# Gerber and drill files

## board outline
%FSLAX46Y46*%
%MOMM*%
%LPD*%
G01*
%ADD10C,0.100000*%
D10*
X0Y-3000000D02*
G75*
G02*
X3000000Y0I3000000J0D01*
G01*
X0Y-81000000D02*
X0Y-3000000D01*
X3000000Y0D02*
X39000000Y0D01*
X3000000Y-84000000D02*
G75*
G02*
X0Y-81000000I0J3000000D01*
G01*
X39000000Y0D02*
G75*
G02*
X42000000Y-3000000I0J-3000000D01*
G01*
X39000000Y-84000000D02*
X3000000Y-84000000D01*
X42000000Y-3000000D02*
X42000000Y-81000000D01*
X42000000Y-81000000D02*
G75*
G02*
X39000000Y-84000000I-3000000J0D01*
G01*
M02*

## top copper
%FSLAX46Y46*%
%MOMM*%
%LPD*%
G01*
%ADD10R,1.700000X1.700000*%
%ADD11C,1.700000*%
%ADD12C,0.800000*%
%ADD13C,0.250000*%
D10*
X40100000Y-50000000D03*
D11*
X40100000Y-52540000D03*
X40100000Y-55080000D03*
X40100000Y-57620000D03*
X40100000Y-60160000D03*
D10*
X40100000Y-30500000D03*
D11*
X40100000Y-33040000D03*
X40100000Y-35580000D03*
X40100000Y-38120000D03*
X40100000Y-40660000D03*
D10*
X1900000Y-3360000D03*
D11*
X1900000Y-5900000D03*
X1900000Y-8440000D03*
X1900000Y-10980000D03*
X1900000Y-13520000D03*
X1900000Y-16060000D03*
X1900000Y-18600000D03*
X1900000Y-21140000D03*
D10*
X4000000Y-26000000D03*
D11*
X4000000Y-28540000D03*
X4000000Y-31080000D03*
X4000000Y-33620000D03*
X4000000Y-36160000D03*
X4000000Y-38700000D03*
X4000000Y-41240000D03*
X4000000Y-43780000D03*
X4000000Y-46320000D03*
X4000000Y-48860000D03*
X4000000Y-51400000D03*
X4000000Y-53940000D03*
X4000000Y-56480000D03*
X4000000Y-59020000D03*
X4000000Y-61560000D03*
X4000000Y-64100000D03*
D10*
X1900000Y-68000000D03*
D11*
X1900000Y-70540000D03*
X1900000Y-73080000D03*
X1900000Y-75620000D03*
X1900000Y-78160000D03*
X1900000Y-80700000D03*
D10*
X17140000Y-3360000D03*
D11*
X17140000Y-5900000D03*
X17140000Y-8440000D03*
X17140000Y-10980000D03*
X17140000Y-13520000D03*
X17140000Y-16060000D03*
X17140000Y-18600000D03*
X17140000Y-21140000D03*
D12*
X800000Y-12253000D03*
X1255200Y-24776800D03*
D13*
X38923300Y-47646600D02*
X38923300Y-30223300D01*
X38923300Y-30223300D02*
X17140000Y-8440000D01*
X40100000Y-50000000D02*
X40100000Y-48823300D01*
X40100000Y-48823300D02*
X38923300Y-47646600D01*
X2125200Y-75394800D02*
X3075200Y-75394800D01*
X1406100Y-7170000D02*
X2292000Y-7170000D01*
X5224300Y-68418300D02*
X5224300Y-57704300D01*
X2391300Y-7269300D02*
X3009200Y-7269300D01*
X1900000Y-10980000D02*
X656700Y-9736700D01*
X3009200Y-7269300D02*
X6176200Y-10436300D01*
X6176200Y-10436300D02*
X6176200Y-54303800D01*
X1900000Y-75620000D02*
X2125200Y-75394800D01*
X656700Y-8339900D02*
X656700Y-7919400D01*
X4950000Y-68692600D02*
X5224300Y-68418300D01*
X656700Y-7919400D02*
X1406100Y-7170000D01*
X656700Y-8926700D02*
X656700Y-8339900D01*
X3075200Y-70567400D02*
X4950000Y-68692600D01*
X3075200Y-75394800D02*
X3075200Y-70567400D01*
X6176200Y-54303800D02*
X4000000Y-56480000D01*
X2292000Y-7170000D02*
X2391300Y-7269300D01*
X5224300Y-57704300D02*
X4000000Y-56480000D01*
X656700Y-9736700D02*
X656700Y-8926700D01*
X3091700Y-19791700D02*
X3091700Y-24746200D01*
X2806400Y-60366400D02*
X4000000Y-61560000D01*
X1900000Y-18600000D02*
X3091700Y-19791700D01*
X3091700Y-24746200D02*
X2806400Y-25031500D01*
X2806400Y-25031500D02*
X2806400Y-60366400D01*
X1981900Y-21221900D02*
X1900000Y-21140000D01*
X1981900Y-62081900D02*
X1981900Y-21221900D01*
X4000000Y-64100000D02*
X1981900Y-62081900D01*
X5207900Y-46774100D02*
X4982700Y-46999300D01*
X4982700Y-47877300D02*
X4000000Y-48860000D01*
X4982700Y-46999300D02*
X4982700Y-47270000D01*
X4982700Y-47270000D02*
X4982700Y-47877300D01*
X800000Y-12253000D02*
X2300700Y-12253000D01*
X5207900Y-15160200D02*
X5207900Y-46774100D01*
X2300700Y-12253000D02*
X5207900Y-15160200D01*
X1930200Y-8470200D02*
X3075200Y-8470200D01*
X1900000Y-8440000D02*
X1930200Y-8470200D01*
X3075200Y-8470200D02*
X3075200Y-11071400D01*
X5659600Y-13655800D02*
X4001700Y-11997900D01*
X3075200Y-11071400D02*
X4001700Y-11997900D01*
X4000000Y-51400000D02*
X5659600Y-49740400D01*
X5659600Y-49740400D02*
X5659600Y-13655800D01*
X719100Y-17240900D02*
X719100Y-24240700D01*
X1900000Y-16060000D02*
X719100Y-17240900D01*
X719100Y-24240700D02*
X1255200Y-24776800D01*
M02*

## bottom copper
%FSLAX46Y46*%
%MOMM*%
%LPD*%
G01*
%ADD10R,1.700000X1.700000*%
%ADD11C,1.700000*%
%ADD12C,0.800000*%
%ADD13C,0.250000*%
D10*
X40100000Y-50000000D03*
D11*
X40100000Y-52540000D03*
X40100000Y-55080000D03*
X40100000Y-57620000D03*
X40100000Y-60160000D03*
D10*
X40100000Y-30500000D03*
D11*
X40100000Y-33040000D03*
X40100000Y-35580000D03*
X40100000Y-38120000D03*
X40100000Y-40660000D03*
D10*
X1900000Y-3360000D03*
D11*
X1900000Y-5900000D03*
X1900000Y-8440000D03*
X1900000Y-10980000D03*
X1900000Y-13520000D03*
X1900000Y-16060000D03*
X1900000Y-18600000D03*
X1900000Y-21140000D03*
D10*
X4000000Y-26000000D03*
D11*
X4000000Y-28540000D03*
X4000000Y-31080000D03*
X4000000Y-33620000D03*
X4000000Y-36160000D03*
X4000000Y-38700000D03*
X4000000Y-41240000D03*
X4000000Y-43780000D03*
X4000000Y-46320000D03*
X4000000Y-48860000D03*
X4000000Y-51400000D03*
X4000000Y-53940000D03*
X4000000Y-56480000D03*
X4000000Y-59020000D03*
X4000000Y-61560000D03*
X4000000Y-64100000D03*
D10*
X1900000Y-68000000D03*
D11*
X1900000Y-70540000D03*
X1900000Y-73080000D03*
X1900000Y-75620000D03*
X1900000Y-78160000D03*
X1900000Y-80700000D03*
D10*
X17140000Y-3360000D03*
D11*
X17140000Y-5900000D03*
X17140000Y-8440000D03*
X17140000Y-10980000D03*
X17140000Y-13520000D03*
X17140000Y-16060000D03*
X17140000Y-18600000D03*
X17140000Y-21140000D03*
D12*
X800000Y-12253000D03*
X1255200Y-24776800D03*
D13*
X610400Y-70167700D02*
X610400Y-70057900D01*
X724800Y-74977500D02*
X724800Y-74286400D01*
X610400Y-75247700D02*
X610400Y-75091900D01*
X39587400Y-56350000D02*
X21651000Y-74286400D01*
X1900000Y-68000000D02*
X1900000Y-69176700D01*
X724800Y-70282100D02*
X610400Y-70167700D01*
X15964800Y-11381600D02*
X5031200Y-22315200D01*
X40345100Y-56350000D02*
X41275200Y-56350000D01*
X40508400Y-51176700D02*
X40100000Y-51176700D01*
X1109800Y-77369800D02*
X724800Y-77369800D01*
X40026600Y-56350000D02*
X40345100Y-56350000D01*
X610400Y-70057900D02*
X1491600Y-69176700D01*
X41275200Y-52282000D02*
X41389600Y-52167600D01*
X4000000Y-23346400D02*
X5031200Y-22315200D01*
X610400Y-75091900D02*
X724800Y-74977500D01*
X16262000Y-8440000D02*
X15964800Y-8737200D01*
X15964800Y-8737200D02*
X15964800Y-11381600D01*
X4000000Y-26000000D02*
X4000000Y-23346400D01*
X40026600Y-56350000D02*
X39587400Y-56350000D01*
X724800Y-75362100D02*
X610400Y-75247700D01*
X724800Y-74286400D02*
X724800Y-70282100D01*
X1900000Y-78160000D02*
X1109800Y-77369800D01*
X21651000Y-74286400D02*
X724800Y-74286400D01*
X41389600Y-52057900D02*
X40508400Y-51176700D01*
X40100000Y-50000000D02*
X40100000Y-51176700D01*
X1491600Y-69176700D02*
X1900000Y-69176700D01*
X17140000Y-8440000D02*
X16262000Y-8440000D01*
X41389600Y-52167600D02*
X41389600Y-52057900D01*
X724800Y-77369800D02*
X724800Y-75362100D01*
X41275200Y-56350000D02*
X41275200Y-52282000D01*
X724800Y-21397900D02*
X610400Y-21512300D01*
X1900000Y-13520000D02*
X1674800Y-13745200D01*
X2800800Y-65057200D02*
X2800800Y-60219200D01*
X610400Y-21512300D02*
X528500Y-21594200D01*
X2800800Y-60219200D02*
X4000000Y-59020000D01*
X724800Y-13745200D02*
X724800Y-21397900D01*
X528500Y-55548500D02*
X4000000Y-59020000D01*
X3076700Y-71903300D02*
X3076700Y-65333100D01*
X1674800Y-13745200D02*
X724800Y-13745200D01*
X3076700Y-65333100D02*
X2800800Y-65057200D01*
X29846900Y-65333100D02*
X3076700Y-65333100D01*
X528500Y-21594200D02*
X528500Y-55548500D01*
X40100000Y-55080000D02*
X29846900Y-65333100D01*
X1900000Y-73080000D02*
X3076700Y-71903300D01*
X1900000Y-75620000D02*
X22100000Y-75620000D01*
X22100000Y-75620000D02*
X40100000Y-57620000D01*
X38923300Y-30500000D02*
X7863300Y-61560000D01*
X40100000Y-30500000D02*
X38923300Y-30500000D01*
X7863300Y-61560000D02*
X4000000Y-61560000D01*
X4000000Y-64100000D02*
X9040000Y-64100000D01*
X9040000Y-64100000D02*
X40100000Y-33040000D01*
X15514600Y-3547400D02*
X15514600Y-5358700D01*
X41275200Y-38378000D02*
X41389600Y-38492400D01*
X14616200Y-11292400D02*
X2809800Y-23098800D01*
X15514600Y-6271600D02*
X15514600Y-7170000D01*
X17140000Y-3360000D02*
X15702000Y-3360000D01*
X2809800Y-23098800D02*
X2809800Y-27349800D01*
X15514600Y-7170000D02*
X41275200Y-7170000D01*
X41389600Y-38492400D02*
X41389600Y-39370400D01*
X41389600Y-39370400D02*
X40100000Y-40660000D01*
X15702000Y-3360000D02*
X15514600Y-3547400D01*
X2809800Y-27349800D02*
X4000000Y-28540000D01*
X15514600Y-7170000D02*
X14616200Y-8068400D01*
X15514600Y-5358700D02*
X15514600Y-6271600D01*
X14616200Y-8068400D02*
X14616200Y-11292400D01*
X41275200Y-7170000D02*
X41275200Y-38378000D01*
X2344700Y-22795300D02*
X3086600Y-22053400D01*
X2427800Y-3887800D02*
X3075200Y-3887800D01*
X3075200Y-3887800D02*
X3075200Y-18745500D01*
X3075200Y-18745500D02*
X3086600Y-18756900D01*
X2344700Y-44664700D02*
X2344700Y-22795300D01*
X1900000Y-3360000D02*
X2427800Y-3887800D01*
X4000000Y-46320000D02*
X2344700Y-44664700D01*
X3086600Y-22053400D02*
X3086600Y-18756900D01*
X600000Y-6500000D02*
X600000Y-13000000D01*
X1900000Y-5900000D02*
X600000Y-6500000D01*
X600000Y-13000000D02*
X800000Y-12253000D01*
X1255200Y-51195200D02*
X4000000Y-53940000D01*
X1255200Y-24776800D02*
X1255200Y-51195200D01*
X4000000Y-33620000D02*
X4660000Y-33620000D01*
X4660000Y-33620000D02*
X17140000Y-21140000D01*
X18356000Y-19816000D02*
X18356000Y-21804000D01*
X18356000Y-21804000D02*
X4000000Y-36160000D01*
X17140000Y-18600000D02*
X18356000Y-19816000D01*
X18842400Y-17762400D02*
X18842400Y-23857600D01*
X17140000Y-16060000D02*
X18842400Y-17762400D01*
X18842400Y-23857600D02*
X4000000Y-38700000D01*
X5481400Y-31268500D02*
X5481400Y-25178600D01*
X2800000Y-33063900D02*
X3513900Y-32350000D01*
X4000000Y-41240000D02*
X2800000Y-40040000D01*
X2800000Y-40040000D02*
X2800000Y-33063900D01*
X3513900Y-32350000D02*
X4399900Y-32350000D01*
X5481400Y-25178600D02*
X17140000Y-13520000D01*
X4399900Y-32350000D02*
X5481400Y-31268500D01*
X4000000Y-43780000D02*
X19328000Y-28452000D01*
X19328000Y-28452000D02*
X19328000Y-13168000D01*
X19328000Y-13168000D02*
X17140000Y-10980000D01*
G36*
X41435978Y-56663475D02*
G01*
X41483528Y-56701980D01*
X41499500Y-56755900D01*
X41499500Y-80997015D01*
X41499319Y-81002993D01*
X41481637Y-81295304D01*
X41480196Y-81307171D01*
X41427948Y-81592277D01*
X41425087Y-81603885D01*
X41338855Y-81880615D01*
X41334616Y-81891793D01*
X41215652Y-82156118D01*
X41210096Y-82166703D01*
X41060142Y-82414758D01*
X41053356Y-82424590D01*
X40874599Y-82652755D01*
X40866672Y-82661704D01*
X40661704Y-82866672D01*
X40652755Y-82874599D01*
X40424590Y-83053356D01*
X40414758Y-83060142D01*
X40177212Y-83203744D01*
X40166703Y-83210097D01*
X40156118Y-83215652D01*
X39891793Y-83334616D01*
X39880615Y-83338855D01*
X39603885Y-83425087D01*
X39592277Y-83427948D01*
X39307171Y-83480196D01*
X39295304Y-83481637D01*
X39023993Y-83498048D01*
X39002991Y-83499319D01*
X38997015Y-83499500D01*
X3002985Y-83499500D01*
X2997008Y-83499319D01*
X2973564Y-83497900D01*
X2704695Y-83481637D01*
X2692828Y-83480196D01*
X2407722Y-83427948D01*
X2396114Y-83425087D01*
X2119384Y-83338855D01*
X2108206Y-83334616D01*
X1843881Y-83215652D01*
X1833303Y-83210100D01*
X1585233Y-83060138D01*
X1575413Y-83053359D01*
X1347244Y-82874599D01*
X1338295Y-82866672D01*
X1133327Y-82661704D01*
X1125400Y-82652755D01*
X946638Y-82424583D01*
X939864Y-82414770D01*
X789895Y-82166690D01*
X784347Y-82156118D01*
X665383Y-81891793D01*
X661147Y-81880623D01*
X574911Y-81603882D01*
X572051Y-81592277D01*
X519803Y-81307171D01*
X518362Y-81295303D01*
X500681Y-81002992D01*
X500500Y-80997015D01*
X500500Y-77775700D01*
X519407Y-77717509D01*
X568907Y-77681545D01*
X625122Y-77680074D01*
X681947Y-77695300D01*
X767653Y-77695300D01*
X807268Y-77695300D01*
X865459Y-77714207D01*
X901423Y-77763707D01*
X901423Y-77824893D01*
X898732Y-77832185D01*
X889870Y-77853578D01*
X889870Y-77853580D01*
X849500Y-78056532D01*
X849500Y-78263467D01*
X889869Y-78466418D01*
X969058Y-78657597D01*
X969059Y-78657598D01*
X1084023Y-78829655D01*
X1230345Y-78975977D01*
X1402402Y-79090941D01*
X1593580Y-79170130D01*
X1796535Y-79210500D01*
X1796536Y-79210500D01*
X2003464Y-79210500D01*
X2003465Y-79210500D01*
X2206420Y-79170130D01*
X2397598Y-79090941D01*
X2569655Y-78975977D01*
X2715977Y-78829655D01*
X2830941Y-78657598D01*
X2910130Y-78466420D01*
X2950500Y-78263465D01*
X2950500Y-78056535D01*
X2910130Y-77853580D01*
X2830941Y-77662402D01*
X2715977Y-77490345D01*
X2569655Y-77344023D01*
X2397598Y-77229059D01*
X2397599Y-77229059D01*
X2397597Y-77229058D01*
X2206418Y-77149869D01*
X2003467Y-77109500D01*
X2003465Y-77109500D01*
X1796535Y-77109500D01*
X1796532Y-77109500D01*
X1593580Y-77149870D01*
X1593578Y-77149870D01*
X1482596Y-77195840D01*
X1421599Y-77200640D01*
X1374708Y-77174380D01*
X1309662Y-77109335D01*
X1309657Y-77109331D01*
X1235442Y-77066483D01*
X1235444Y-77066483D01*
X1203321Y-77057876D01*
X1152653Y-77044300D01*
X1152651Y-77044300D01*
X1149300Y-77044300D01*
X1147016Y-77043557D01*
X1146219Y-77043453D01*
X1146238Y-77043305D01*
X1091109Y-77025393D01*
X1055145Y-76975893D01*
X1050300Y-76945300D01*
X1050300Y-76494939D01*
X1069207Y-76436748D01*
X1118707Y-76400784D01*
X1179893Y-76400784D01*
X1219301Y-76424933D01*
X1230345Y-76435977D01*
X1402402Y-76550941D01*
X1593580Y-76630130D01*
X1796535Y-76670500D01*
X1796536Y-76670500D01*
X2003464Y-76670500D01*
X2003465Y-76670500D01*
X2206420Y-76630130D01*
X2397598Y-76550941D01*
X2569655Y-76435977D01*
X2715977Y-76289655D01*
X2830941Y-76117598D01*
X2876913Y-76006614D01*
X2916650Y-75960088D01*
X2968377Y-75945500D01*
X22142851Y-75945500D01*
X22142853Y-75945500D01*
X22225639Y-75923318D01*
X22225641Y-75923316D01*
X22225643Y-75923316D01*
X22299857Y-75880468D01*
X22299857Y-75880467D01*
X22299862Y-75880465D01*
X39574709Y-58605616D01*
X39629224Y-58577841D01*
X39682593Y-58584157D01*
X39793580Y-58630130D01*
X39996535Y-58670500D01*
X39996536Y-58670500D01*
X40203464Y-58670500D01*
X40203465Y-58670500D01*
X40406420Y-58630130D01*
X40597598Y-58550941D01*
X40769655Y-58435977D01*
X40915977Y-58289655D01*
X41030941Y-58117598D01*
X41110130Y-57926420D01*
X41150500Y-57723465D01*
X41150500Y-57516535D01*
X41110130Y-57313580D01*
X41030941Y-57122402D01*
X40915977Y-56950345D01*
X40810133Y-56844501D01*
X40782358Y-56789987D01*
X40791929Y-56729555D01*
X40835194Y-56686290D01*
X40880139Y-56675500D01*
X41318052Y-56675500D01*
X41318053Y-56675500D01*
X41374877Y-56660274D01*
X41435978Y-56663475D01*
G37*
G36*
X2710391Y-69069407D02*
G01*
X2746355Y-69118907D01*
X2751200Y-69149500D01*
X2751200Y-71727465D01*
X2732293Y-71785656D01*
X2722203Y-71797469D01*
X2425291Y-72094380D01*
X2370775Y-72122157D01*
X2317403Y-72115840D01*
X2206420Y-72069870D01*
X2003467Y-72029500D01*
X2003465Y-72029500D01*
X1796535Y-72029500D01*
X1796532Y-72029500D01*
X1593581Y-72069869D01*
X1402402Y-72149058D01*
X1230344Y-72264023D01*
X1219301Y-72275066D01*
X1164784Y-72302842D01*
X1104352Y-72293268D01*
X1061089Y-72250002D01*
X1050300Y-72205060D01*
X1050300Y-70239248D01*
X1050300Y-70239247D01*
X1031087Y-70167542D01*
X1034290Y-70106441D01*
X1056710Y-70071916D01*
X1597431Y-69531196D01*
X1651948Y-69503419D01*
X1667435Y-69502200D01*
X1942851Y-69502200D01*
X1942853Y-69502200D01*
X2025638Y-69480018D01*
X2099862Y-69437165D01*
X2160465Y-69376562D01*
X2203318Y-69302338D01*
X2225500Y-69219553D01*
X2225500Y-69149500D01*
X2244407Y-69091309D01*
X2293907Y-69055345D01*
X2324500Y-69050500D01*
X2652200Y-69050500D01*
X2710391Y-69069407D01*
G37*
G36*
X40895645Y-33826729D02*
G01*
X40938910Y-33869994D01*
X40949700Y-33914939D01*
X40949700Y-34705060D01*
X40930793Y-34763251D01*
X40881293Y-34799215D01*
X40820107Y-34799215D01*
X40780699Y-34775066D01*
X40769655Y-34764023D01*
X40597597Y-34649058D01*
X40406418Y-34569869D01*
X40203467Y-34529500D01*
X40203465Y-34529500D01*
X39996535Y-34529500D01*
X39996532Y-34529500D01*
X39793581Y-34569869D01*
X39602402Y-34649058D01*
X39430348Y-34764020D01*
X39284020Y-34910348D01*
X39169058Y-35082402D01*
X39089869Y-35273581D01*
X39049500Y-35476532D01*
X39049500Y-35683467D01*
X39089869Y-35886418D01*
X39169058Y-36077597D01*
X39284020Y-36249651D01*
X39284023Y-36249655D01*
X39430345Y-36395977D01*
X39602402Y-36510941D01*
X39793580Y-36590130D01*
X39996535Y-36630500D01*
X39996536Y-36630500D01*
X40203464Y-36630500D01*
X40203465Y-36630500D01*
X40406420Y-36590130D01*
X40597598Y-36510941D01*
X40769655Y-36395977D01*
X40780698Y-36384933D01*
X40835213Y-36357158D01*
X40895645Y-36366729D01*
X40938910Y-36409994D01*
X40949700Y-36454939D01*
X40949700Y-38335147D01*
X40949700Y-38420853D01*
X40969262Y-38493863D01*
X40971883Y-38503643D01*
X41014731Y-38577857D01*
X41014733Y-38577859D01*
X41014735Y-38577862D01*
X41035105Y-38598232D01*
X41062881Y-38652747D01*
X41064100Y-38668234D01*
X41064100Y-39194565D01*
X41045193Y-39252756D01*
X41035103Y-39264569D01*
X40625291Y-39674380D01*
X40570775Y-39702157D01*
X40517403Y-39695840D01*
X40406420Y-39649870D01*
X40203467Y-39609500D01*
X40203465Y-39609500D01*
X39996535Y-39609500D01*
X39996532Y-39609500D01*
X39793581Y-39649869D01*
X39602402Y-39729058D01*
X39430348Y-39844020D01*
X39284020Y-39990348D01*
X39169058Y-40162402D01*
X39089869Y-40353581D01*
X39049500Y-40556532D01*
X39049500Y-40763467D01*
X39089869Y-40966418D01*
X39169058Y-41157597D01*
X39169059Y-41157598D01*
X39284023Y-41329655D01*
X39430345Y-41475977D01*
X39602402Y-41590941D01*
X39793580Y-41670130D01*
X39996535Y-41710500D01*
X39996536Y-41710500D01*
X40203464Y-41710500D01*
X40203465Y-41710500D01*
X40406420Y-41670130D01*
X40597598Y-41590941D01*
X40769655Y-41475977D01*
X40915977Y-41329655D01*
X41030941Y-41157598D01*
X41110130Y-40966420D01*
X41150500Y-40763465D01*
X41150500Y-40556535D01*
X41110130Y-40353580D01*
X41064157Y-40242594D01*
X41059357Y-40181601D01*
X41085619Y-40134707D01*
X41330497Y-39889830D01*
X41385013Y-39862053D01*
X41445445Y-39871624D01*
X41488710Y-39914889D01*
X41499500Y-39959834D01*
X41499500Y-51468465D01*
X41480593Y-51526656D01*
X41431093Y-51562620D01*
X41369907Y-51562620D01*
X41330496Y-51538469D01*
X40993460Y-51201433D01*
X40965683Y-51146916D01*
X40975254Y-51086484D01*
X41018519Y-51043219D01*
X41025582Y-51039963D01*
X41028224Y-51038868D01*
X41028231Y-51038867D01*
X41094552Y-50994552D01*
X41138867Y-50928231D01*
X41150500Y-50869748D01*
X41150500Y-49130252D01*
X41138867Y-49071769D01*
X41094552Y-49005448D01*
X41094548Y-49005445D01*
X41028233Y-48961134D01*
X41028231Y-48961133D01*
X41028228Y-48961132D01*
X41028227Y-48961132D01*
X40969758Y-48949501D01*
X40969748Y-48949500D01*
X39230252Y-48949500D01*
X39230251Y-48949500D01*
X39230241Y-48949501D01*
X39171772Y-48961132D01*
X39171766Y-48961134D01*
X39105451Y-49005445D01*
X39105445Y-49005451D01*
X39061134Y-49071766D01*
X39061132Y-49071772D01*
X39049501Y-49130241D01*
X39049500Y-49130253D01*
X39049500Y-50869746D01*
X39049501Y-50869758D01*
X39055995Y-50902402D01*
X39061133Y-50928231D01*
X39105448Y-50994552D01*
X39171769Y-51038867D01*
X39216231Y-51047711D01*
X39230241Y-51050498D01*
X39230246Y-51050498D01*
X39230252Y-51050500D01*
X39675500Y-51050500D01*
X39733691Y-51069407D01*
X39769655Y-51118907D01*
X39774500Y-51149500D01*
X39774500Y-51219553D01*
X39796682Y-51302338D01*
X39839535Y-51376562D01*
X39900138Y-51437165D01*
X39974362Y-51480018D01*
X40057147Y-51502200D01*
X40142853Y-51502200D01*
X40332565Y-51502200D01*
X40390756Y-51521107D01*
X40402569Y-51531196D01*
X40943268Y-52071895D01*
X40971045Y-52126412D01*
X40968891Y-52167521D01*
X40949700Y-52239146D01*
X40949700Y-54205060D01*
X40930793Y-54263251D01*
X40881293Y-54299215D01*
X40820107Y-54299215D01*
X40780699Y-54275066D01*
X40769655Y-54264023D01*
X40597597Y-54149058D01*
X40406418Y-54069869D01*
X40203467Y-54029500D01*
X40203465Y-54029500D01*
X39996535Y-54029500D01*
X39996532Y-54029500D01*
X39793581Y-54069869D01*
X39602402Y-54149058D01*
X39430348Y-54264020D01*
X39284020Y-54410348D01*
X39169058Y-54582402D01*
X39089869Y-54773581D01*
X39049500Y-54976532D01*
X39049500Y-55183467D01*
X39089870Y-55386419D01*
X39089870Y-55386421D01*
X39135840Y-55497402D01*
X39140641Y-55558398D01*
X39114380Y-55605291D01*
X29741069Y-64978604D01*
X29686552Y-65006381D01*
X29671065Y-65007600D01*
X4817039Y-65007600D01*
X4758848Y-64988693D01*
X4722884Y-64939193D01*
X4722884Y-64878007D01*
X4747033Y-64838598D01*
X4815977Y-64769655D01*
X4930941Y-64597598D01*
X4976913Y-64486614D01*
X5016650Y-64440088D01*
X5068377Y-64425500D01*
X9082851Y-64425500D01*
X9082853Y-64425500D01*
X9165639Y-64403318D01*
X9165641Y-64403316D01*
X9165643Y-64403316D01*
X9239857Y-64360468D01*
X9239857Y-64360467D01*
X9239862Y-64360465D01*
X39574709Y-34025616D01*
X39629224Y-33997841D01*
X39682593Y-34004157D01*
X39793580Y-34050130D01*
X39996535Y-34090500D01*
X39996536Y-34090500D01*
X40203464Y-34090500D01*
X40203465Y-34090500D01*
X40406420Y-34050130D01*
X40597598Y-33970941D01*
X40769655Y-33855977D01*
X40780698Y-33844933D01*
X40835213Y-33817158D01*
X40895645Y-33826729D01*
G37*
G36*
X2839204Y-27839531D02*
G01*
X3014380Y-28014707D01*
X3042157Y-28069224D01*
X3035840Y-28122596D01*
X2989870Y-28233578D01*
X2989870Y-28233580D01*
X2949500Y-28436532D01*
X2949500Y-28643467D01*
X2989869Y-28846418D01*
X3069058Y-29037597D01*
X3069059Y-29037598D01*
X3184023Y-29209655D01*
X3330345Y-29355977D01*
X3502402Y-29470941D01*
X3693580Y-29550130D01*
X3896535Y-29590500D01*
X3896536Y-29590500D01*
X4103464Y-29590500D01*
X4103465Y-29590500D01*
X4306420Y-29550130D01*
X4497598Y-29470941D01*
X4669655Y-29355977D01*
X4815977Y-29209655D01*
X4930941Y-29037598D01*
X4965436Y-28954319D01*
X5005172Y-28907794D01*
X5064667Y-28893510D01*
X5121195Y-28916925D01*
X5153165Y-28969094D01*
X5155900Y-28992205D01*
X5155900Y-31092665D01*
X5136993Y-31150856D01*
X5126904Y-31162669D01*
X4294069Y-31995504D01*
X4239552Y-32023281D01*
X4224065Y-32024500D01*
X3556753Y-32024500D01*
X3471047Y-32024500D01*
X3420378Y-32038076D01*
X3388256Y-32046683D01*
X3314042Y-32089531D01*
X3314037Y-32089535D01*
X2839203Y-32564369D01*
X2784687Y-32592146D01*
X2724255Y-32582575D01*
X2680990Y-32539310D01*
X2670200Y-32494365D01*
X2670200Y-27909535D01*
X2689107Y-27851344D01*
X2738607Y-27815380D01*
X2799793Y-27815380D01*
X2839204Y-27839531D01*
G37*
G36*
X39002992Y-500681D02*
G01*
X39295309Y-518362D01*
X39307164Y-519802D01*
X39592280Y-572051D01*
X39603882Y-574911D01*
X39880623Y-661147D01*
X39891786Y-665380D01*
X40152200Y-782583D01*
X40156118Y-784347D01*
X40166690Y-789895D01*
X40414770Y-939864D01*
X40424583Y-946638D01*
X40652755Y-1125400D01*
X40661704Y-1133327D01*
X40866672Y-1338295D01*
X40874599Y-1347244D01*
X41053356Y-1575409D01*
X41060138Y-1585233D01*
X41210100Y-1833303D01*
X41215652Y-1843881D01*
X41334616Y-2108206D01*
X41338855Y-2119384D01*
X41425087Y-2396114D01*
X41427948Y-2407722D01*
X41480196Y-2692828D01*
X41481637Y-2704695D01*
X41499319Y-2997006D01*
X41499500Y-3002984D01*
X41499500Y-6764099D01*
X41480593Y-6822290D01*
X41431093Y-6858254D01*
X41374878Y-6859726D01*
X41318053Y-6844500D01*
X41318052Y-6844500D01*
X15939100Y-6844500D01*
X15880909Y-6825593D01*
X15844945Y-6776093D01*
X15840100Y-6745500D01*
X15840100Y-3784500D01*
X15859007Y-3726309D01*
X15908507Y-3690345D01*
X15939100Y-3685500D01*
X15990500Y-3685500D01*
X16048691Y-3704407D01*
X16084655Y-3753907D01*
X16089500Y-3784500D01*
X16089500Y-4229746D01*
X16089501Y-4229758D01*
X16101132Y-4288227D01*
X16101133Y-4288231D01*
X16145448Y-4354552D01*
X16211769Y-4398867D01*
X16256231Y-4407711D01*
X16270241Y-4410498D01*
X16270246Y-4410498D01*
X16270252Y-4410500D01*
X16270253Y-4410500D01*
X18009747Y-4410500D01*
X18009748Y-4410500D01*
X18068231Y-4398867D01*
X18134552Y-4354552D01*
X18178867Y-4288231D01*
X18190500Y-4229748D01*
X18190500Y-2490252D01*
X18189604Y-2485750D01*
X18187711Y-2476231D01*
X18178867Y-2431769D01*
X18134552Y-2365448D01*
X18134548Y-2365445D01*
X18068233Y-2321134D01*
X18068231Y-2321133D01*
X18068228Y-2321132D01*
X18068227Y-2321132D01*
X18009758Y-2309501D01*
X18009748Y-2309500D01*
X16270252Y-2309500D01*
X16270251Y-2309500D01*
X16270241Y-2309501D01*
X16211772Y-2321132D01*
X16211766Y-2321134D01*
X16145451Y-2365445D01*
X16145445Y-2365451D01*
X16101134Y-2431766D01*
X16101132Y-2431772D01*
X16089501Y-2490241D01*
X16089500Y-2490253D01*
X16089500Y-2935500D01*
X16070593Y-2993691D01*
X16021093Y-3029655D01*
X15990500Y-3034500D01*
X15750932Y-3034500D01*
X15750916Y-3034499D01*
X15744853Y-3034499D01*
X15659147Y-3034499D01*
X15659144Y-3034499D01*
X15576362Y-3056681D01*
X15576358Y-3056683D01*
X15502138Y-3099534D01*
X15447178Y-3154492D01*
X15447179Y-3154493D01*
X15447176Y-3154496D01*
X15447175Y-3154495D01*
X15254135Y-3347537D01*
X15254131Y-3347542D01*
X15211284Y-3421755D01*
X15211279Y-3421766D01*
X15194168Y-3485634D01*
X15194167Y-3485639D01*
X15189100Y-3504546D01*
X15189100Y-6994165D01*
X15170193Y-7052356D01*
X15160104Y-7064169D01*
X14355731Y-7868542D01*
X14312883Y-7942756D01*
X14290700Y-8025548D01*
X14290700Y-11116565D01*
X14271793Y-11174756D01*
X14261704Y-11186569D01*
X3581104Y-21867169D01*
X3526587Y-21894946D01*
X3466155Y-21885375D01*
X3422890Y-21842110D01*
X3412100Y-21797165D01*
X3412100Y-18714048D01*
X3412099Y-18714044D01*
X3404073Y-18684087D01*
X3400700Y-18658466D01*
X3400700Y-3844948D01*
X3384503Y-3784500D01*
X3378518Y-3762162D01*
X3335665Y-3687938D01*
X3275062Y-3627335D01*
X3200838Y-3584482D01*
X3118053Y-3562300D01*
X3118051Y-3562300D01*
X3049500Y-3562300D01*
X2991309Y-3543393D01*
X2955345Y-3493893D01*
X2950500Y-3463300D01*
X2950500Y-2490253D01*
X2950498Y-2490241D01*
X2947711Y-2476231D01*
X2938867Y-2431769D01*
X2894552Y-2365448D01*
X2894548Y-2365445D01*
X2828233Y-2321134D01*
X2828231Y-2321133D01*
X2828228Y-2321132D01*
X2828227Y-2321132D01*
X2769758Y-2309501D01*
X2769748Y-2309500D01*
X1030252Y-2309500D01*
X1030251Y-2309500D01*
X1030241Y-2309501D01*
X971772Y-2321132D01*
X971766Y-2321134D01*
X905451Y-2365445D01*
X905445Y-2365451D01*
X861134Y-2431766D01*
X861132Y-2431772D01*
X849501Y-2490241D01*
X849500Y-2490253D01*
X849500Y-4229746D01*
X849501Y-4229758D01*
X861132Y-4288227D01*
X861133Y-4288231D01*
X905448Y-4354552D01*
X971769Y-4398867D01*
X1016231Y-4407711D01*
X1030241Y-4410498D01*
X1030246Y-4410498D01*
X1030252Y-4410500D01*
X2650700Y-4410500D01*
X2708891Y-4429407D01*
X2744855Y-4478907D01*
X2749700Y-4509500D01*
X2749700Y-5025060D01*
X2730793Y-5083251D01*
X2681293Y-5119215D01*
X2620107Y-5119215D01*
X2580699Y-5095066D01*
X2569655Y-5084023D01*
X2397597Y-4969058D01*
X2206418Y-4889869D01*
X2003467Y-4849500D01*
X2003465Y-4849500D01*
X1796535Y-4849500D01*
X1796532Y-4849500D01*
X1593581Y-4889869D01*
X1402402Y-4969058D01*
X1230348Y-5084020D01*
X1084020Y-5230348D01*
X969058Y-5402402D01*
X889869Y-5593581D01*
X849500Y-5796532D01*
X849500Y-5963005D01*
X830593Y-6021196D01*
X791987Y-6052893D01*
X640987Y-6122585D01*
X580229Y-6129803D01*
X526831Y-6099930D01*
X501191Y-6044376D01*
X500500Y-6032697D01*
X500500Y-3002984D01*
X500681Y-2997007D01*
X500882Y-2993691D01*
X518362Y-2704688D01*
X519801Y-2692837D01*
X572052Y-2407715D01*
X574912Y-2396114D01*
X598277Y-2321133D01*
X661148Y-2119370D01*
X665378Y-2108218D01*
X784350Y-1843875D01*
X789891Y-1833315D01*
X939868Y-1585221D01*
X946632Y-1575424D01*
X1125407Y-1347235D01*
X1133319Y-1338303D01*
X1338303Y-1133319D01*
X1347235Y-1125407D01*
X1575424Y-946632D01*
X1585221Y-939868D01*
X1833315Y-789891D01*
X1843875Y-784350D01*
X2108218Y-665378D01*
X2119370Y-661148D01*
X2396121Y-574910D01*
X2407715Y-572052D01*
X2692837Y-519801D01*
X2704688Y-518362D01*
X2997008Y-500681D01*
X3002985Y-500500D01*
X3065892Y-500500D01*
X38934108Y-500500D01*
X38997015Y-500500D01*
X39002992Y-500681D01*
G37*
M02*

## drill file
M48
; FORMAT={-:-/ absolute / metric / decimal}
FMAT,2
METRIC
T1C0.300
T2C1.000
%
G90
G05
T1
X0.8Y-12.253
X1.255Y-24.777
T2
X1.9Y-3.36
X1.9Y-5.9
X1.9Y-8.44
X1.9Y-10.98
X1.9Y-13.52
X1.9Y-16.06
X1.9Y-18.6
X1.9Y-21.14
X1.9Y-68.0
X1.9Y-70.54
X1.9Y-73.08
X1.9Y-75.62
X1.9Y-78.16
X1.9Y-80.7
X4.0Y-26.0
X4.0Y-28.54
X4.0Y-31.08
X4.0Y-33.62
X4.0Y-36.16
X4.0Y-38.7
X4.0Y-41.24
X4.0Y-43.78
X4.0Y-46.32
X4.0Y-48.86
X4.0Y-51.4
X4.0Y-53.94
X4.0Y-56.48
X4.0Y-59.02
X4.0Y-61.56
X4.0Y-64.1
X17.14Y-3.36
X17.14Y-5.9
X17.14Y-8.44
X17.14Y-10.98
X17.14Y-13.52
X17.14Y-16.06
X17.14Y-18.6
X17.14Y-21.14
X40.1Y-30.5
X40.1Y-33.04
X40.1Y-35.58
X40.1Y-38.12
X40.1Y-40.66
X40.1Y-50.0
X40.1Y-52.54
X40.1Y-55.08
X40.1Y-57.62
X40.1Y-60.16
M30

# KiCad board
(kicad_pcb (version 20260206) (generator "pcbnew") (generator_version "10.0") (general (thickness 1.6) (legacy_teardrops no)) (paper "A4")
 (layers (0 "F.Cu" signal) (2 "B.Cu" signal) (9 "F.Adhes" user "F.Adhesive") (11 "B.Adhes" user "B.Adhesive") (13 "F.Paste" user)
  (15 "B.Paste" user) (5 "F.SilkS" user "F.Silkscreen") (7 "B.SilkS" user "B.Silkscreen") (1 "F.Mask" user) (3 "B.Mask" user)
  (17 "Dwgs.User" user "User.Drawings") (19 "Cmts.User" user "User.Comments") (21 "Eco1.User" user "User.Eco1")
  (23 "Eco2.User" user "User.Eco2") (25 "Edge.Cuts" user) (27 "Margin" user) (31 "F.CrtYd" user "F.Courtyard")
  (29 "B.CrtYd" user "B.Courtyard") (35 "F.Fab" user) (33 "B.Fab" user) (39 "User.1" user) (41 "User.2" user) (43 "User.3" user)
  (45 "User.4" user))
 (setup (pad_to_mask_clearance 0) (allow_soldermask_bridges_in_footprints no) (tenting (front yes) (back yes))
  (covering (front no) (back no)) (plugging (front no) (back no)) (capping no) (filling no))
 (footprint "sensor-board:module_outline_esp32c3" (layer "F.Cu") (at 21 12.25)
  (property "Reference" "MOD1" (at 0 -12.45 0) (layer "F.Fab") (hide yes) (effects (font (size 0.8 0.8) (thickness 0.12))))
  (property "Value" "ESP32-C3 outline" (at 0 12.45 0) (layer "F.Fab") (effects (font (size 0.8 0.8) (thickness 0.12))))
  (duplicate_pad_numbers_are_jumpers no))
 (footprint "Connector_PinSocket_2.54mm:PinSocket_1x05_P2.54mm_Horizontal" (layer "F.Cu") (at 40.1 50)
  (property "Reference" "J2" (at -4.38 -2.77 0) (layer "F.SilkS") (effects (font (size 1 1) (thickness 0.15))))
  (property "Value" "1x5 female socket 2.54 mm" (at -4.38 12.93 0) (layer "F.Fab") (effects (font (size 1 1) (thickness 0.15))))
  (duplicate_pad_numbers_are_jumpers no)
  (pad "1" thru_hole rect (at 0 0) (size 1.7 1.7) (drill 1) (layers "*.Cu" "*.Mask") (remove_unused_layers no) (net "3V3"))
  (pad "2" thru_hole circle (at 0 2.54) (size 1.7 1.7) (drill 1) (layers "*.Cu" "*.Mask") (remove_unused_layers no) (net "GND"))
  (pad "3" thru_hole circle (at 0 5.08) (size 1.7 1.7) (drill 1) (layers "*.Cu" "*.Mask") (remove_unused_layers no) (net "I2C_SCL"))
  (pad "4" thru_hole circle (at 0 7.62) (size 1.7 1.7) (drill 1) (layers "*.Cu" "*.Mask") (remove_unused_layers no) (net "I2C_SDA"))
  (pad "5" thru_hole circle (at 0 10.16) (size 1.7 1.7) (drill 1) (layers "*.Cu" "*.Mask") (remove_unused_layers no) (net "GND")))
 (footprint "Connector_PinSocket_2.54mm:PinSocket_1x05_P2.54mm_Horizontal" (layer "F.Cu") (at 40.1 30.5)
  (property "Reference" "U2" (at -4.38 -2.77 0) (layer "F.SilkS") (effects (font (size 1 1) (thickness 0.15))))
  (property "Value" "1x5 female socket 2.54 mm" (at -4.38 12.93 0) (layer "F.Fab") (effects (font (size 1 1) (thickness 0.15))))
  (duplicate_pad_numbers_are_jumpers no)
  (pad "1" thru_hole rect (at 0 0) (size 1.7 1.7) (drill 1) (layers "*.Cu" "*.Mask") (remove_unused_layers no) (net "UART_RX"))
  (pad "2" thru_hole circle (at 0 2.54) (size 1.7 1.7) (drill 1) (layers "*.Cu" "*.Mask") (remove_unused_layers no) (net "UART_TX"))
  (pad "3" thru_hole circle (at 0 5.08) (size 1.7 1.7) (drill 1) (layers "*.Cu" "*.Mask") (remove_unused_layers no))
  (pad "4" thru_hole circle (at 0 7.62) (size 1.7 1.7) (drill 1) (layers "*.Cu" "*.Mask") (remove_unused_layers no) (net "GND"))
  (pad "5" thru_hole circle (at 0 10.16) (size 1.7 1.7) (drill 1) (layers "*.Cu" "*.Mask") (remove_unused_layers no) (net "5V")))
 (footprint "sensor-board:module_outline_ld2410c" (layer "F.Cu") (at 23.16 35.58)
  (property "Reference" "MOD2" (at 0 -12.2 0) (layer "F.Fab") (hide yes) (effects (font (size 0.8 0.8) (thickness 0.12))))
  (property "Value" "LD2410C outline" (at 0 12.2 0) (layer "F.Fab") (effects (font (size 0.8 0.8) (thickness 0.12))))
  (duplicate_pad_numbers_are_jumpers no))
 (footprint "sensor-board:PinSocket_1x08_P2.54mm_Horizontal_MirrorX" (layer "F.Cu") (at 1.9 3.36)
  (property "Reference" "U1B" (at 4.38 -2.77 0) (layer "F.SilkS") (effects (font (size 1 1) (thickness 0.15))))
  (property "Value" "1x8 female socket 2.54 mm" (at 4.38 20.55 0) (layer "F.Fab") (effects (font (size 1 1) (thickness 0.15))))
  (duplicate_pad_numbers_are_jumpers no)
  (pad "1" thru_hole rect (at 0 0) (size 1.7 1.7) (drill 1) (layers "*.Cu" "*.Mask") (remove_unused_layers no) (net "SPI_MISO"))
  (pad "2" thru_hole circle (at 0 2.54) (size 1.7 1.7) (drill 1) (layers "*.Cu" "*.Mask") (remove_unused_layers no) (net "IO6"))
  (pad "3" thru_hole circle (at 0 5.08) (size 1.7 1.7) (drill 1) (layers "*.Cu" "*.Mask") (remove_unused_layers no) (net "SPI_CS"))
  (pad "4" thru_hole circle (at 0 7.62) (size 1.7 1.7) (drill 1) (layers "*.Cu" "*.Mask") (remove_unused_layers no) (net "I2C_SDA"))
  (pad "5" thru_hole circle (at 0 10.16) (size 1.7 1.7) (drill 1) (layers "*.Cu" "*.Mask") (remove_unused_layers no) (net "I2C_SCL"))
  (pad "6" thru_hole circle (at 0 12.7) (size 1.7 1.7) (drill 1) (layers "*.Cu" "*.Mask") (remove_unused_layers no) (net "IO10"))
  (pad "7" thru_hole circle (at 0 15.24) (size 1.7 1.7) (drill 1) (layers "*.Cu" "*.Mask") (remove_unused_layers no) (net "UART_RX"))
  (pad "8" thru_hole circle (at 0 17.78) (size 1.7 1.7) (drill 1) (layers "*.Cu" "*.Mask") (remove_unused_layers no) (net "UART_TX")))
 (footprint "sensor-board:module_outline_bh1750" (layer "F.Cu") (at 21 54.955)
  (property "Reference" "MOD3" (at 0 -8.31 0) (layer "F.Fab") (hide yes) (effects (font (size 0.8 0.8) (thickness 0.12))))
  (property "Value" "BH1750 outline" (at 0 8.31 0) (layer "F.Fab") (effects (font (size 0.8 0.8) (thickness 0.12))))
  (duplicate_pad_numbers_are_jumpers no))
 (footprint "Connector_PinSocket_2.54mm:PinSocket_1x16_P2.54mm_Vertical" (layer "F.Cu") (at 4 26)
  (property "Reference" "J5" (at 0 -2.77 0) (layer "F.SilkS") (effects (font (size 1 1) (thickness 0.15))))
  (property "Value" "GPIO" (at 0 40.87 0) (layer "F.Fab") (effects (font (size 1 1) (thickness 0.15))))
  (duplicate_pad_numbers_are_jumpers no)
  (pad "1" thru_hole rect (at 0 0) (size 1.7 1.7) (drill 1) (layers "*.Cu" "*.Mask") (remove_unused_layers no) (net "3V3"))
  (pad "2" thru_hole circle (at 0 2.54) (size 1.7 1.7) (drill 1) (layers "*.Cu" "*.Mask") (remove_unused_layers no) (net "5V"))
  (pad "3" thru_hole circle (at 0 5.08) (size 1.7 1.7) (drill 1) (layers "*.Cu" "*.Mask") (remove_unused_layers no) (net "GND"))
  (pad "4" thru_hole circle (at 0 7.62) (size 1.7 1.7) (drill 1) (layers "*.Cu" "*.Mask") (remove_unused_layers no) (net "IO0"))
  (pad "5" thru_hole circle (at 0 10.16) (size 1.7 1.7) (drill 1) (layers "*.Cu" "*.Mask") (remove_unused_layers no) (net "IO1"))
  (pad "6" thru_hole circle (at 0 12.7) (size 1.7 1.7) (drill 1) (layers "*.Cu" "*.Mask") (remove_unused_layers no) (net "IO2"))
  (pad "7" thru_hole circle (at 0 15.24) (size 1.7 1.7) (drill 1) (layers "*.Cu" "*.Mask") (remove_unused_layers no) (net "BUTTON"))
  (pad "8" thru_hole circle (at 0 17.78) (size 1.7 1.7) (drill 1) (layers "*.Cu" "*.Mask") (remove_unused_layers no) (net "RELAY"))
  (pad "9" thru_hole circle (at 0 20.32) (size 1.7 1.7) (drill 1) (layers "*.Cu" "*.Mask") (remove_unused_layers no) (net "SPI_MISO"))
  (pad "10" thru_hole circle (at 0 22.86) (size 1.7 1.7) (drill 1) (layers "*.Cu" "*.Mask") (remove_unused_layers no) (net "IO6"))
  (pad "11" thru_hole circle (at 0 25.4) (size 1.7 1.7) (drill 1) (layers "*.Cu" "*.Mask") (remove_unused_layers no) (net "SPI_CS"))
  (pad "12" thru_hole circle (at 0 27.94) (size 1.7 1.7) (drill 1) (layers "*.Cu" "*.Mask") (remove_unused_layers no) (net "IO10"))
  (pad "13" thru_hole circle (at 0 30.48) (size 1.7 1.7) (drill 1) (layers "*.Cu" "*.Mask") (remove_unused_layers no) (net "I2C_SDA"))
  (pad "14" thru_hole circle (at 0 33.02) (size 1.7 1.7) (drill 1) (layers "*.Cu" "*.Mask") (remove_unused_layers no) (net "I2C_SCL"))
  (pad "15" thru_hole circle (at 0 35.56) (size 1.7 1.7) (drill 1) (layers "*.Cu" "*.Mask") (remove_unused_layers no) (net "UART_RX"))
  (pad "16" thru_hole circle (at 0 38.1) (size 1.7 1.7) (drill 1) (layers "*.Cu" "*.Mask") (remove_unused_layers no) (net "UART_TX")))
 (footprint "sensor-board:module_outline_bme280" (layer "F.Cu") (at 18.33 73.475)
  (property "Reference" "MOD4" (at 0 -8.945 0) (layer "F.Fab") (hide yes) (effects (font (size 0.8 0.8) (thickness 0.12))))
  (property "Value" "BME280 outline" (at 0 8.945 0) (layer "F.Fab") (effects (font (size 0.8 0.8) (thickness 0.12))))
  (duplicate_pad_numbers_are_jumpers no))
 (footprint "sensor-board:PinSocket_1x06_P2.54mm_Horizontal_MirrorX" (layer "F.Cu") (at 1.9 68)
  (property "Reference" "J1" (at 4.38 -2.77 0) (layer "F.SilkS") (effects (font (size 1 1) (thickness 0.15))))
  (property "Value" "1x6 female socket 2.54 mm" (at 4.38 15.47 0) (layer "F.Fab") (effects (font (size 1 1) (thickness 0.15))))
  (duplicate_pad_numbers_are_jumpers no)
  (pad "1" thru_hole rect (at 0 0) (size 1.7 1.7) (drill 1) (layers "*.Cu" "*.Mask") (remove_unused_layers no) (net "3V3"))
  (pad "2" thru_hole circle (at 0 2.54) (size 1.7 1.7) (drill 1) (layers "*.Cu" "*.Mask") (remove_unused_layers no) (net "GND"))
  (pad "3" thru_hole circle (at 0 5.08) (size 1.7 1.7) (drill 1) (layers "*.Cu" "*.Mask") (remove_unused_layers no) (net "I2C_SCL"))
  (pad "4" thru_hole circle (at 0 7.62) (size 1.7 1.7) (drill 1) (layers "*.Cu" "*.Mask") (remove_unused_layers no) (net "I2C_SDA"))
  (pad "5" thru_hole circle (at 0 10.16) (size 1.7 1.7) (drill 1) (layers "*.Cu" "*.Mask") (remove_unused_layers no) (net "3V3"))
  (pad "6" thru_hole circle (at 0 12.7) (size 1.7 1.7) (drill 1) (layers "*.Cu" "*.Mask") (remove_unused_layers no) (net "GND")))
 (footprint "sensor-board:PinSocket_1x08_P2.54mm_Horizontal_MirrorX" (layer "F.Cu") (at 17.14 3.36)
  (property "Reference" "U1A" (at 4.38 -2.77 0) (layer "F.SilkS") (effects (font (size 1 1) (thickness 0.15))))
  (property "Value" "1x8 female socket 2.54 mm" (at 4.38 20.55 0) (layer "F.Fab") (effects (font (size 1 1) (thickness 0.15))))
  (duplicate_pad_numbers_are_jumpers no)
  (pad "1" thru_hole rect (at 0 0) (size 1.7 1.7) (drill 1) (layers "*.Cu" "*.Mask") (remove_unused_layers no) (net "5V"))
  (pad "2" thru_hole circle (at 0 2.54) (size 1.7 1.7) (drill 1) (layers "*.Cu" "*.Mask") (remove_unused_layers no) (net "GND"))
  (pad "3" thru_hole circle (at 0 5.08) (size 1.7 1.7) (drill 1) (layers "*.Cu" "*.Mask") (remove_unused_layers no) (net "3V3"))
  (pad "4" thru_hole circle (at 0 7.62) (size 1.7 1.7) (drill 1) (layers "*.Cu" "*.Mask") (remove_unused_layers no) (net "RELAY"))
  (pad "5" thru_hole circle (at 0 10.16) (size 1.7 1.7) (drill 1) (layers "*.Cu" "*.Mask") (remove_unused_layers no) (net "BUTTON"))
  (pad "6" thru_hole circle (at 0 12.7) (size 1.7 1.7) (drill 1) (layers "*.Cu" "*.Mask") (remove_unused_layers no) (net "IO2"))
  (pad "7" thru_hole circle (at 0 15.24) (size 1.7 1.7) (drill 1) (layers "*.Cu" "*.Mask") (remove_unused_layers no) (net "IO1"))
  (pad "8" thru_hole circle (at 0 17.78) (size 1.7 1.7) (drill 1) (layers "*.Cu" "*.Mask") (remove_unused_layers no) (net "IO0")))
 (gr_arc (start 0 3) (mid 0.87868 0.87868) (end 3 0) (stroke (width 0.1) (type default)) (layer "Edge.Cuts"))
 (gr_line (start 0 81) (end 0 3) (stroke (width 0.1) (type default)) (layer "Edge.Cuts"))
 (gr_line (start 3 0) (end 39 0) (stroke (width 0.1) (type default)) (layer "Edge.Cuts"))
 (gr_arc (start 3 84) (mid 0.87868 83.12132) (end 0 81) (stroke (width 0.1) (type default)) (layer "Edge.Cuts"))
 (gr_arc (start 39 0) (mid 41.12132 0.87868) (end 42 3) (stroke (width 0.1) (type default)) (layer "Edge.Cuts"))
 (gr_line (start 39 84) (end 3 84) (stroke (width 0.1) (type default)) (layer "Edge.Cuts"))
 (gr_line (start 42 3) (end 42 81) (stroke (width 0.1) (type default)) (layer "Edge.Cuts"))
 (gr_arc (start 42 81) (mid 41.12132 83.12132) (end 39 84) (stroke (width 0.1) (type default)) (layer "Edge.Cuts"))
 (segment (start 38.9233 47.6466) (end 38.9233 30.2233) (width 0.25) (layer "F.Cu") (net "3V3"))
 (segment (start 38.9233 30.2233) (end 17.14 8.44) (width 0.25) (layer "F.Cu") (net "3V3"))
 (segment (start 40.1 50) (end 40.1 48.8233) (width 0.25) (layer "F.Cu") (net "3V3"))
 (segment (start 40.1 48.8233) (end 38.9233 47.6466) (width 0.25) (layer "F.Cu") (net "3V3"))
 (segment (start 0.6104 70.1677) (end 0.6104 70.0579) (width 0.25) (layer "B.Cu") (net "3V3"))
 (segment (start 0.7248 74.9775) (end 0.7248 74.2864) (width 0.25) (layer "B.Cu") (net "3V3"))
 (segment (start 0.6104 75.2477) (end 0.6104 75.0919) (width 0.25) (layer "B.Cu") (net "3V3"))
 (segment (start 39.5874 56.35) (end 21.651 74.2864) (width 0.25) (layer "B.Cu") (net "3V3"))
 (segment (start 1.9 68) (end 1.9 69.1767) (width 0.25) (layer "B.Cu") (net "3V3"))
 (segment (start 0.7248 70.2821) (end 0.6104 70.1677) (width 0.25) (layer "B.Cu") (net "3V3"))
 (segment (start 15.9648 11.3816) (end 5.0312 22.3152) (width 0.25) (layer "B.Cu") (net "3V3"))
 (segment (start 40.3451 56.35) (end 41.2752 56.35) (width 0.25) (layer "B.Cu") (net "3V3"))
 (segment (start 40.5084 51.1767) (end 40.1 51.1767) (width 0.25) (layer "B.Cu") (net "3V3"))
 (segment (start 1.1098 77.3698) (end 0.7248 77.3698) (width 0.25) (layer "B.Cu") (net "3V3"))
 (segment (start 40.0266 56.35) (end 40.3451 56.35) (width 0.25) (layer "B.Cu") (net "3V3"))
 (segment (start 0.6104 70.0579) (end 1.4916 69.1767) (width 0.25) (layer "B.Cu") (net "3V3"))
 (segment (start 41.2752 52.282) (end 41.3896 52.1676) (width 0.25) (layer "B.Cu") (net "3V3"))
 (segment (start 4 23.3464) (end 5.0312 22.3152) (width 0.25) (layer "B.Cu") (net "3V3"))
 (segment (start 0.6104 75.0919) (end 0.7248 74.9775) (width 0.25) (layer "B.Cu") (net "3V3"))
 (segment (start 16.262 8.44) (end 15.9648 8.7372) (width 0.25) (layer "B.Cu") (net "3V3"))
 (segment (start 15.9648 8.7372) (end 15.9648 11.3816) (width 0.25) (layer "B.Cu") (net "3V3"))
 (segment (start 4 26) (end 4 23.3464) (width 0.25) (layer "B.Cu") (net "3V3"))
 (segment (start 40.0266 56.35) (end 39.5874 56.35) (width 0.25) (layer "B.Cu") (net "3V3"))
 (segment (start 0.7248 75.3621) (end 0.6104 75.2477) (width 0.25) (layer "B.Cu") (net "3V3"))
 (segment (start 0.7248 74.2864) (end 0.7248 70.2821) (width 0.25) (layer "B.Cu") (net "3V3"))
 (segment (start 1.9 78.16) (end 1.1098 77.3698) (width 0.25) (layer "B.Cu") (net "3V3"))
 (segment (start 21.651 74.2864) (end 0.7248 74.2864) (width 0.25) (layer "B.Cu") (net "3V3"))
 (segment (start 41.3896 52.0579) (end 40.5084 51.1767) (width 0.25) (layer "B.Cu") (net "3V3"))
 (segment (start 40.1 50) (end 40.1 51.1767) (width 0.25) (layer "B.Cu") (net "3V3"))
 (segment (start 1.4916 69.1767) (end 1.9 69.1767) (width 0.25) (layer "B.Cu") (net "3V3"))
 (segment (start 17.14 8.44) (end 16.262 8.44) (width 0.25) (layer "B.Cu") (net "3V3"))
 (segment (start 41.3896 52.1676) (end 41.3896 52.0579) (width 0.25) (layer "B.Cu") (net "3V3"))
 (segment (start 0.7248 77.3698) (end 0.7248 75.3621) (width 0.25) (layer "B.Cu") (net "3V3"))
 (segment (start 41.2752 56.35) (end 41.2752 52.282) (width 0.25) (layer "B.Cu") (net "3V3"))
 (segment (start 0.7248 21.3979) (end 0.6104 21.5123) (width 0.25) (layer "B.Cu") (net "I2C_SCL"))
 (segment (start 1.9 13.52) (end 1.6748 13.7452) (width 0.25) (layer "B.Cu") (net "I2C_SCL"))
 (segment (start 2.8008 65.0572) (end 2.8008 60.2192) (width 0.25) (layer "B.Cu") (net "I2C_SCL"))
 (segment (start 0.6104 21.5123) (end 0.5285 21.5942) (width 0.25) (layer "B.Cu") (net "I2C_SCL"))
 (segment (start 2.8008 60.2192) (end 4 59.02) (width 0.25) (layer "B.Cu") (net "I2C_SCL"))
 (segment (start 0.7248 13.7452) (end 0.7248 21.3979) (width 0.25) (layer "B.Cu") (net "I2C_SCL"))
 (segment (start 0.5285 55.5485) (end 4 59.02) (width 0.25) (layer "B.Cu") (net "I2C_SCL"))
 (segment (start 3.0767 71.9033) (end 3.0767 65.3331) (width 0.25) (layer "B.Cu") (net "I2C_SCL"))
 (segment (start 1.6748 13.7452) (end 0.7248 13.7452) (width 0.25) (layer "B.Cu") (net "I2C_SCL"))
 (segment (start 3.0767 65.3331) (end 2.8008 65.0572) (width 0.25) (layer "B.Cu") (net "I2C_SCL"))
 (segment (start 29.8469 65.3331) (end 3.0767 65.3331) (width 0.25) (layer "B.Cu") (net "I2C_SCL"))
 (segment (start 0.5285 21.5942) (end 0.5285 55.5485) (width 0.25) (layer "B.Cu") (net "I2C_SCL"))
 (segment (start 40.1 55.08) (end 29.8469 65.3331) (width 0.25) (layer "B.Cu") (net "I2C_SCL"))
 (segment (start 1.9 73.08) (end 3.0767 71.9033) (width 0.25) (layer "B.Cu") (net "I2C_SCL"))
 (segment (start 2.1252 75.3948) (end 3.0752 75.3948) (width 0.25) (layer "F.Cu") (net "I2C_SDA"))
 (segment (start 1.4061 7.17) (end 2.292 7.17) (width 0.25) (layer "F.Cu") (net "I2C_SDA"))
 (segment (start 5.2243 68.4183) (end 5.2243 57.7043) (width 0.25) (layer "F.Cu") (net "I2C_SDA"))
 (segment (start 2.3913 7.2693) (end 3.0092 7.2693) (width 0.25) (layer "F.Cu") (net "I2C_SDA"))
 (segment (start 1.9 10.98) (end 0.6567 9.7367) (width 0.25) (layer "F.Cu") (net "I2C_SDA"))
 (segment (start 3.0092 7.2693) (end 6.1762 10.4363) (width 0.25) (layer "F.Cu") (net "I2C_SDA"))
 (segment (start 6.1762 10.4363) (end 6.1762 54.3038) (width 0.25) (layer "F.Cu") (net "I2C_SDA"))
 (segment (start 1.9 75.62) (end 2.1252 75.3948) (width 0.25) (layer "F.Cu") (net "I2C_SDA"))
 (segment (start 0.6567 8.3399) (end 0.6567 7.9194) (width 0.25) (layer "F.Cu") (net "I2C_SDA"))
 (segment (start 4.95 68.6926) (end 5.2243 68.4183) (width 0.25) (layer "F.Cu") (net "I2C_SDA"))
 (segment (start 0.6567 7.9194) (end 1.4061 7.17) (width 0.25) (layer "F.Cu") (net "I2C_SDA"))
 (segment (start 0.6567 8.9267) (end 0.6567 8.3399) (width 0.25) (layer "F.Cu") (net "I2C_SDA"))
 (segment (start 3.0752 70.5674) (end 4.95 68.6926) (width 0.25) (layer "F.Cu") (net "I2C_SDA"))
 (segment (start 3.0752 75.3948) (end 3.0752 70.5674) (width 0.25) (layer "F.Cu") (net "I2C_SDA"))
 (segment (start 6.1762 54.3038) (end 4 56.48) (width 0.25) (layer "F.Cu") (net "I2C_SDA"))
 (segment (start 2.292 7.17) (end 2.3913 7.2693) (width 0.25) (layer "F.Cu") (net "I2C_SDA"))
 (segment (start 5.2243 57.7043) (end 4 56.48) (width 0.25) (layer "F.Cu") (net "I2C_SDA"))
 (segment (start 0.6567 9.7367) (end 0.6567 8.9267) (width 0.25) (layer "F.Cu") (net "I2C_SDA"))
 (segment (start 1.9 75.62) (end 22.1 75.62) (width 0.25) (layer "B.Cu") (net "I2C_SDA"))
 (segment (start 22.1 75.62) (end 40.1 57.62) (width 0.25) (layer "B.Cu") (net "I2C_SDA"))
 (segment (start 3.0917 19.7917) (end 3.0917 24.7462) (width 0.25) (layer "F.Cu") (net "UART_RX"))
 (segment (start 2.8064 60.3664) (end 4 61.56) (width 0.25) (layer "F.Cu") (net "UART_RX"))
 (segment (start 1.9 18.6) (end 3.0917 19.7917) (width 0.25) (layer "F.Cu") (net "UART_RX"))
 (segment (start 3.0917 24.7462) (end 2.8064 25.0315) (width 0.25) (layer "F.Cu") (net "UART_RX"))
 (segment (start 2.8064 25.0315) (end 2.8064 60.3664) (width 0.25) (layer "F.Cu") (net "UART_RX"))
 (segment (start 38.9233 30.5) (end 7.8633 61.56) (width 0.25) (layer "B.Cu") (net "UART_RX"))
 (segment (start 40.1 30.5) (end 38.9233 30.5) (width 0.25) (layer "B.Cu") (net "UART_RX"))
 (segment (start 7.8633 61.56) (end 4 61.56) (width 0.25) (layer "B.Cu") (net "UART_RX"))
 (segment (start 1.9819 21.2219) (end 1.9 21.14) (width 0.25) (layer "F.Cu") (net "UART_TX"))
 (segment (start 1.9819 62.0819) (end 1.9819 21.2219) (width 0.25) (layer "F.Cu") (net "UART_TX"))
 (segment (start 4 64.1) (end 1.9819 62.0819) (width 0.25) (layer "F.Cu") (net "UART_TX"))
 (segment (start 4 64.1) (end 9.04 64.1) (width 0.25) (layer "B.Cu") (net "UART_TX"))
 (segment (start 9.04 64.1) (end 40.1 33.04) (width 0.25) (layer "B.Cu") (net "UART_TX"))
 (segment (start 15.5146 3.5474) (end 15.5146 5.3587) (width 0.25) (layer "B.Cu") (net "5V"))
 (segment (start 41.2752 38.378) (end 41.3896 38.4924) (width 0.25) (layer "B.Cu") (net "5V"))
 (segment (start 14.6162 11.2924) (end 2.8098 23.0988) (width 0.25) (layer "B.Cu") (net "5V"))
 (segment (start 15.5146 6.2716) (end 15.5146 7.17) (width 0.25) (layer "B.Cu") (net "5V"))
 (segment (start 17.14 3.36) (end 15.702 3.36) (width 0.25) (layer "B.Cu") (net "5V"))
 (segment (start 2.8098 23.0988) (end 2.8098 27.3498) (width 0.25) (layer "B.Cu") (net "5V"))
 (segment (start 15.5146 7.17) (end 41.2752 7.17) (width 0.25) (layer "B.Cu") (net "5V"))
 (segment (start 41.3896 38.4924) (end 41.3896 39.3704) (width 0.25) (layer "B.Cu") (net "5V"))
 (segment (start 41.3896 39.3704) (end 40.1 40.66) (width 0.25) (layer "B.Cu") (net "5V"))
 (segment (start 15.702 3.36) (end 15.5146 3.5474) (width 0.25) (layer "B.Cu") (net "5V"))
 (segment (start 2.8098 27.3498) (end 4 28.54) (width 0.25) (layer "B.Cu") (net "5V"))
 (segment (start 15.5146 7.17) (end 14.6162 8.0684) (width 0.25) (layer "B.Cu") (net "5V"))
 (segment (start 15.5146 5.3587) (end 15.5146 6.2716) (width 0.25) (layer "B.Cu") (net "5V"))
 (segment (start 14.6162 8.0684) (end 14.6162 11.2924) (width 0.25) (layer "B.Cu") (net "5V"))
 (segment (start 41.2752 7.17) (end 41.2752 38.378) (width 0.25) (layer "B.Cu") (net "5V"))
 (segment (start 2.3447 22.7953) (end 3.0866 22.0534) (width 0.25) (layer "B.Cu") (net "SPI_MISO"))
 (segment (start 2.4278 3.8878) (end 3.0752 3.8878) (width 0.25) (layer "B.Cu") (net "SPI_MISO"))
 (segment (start 3.0752 3.8878) (end 3.0752 18.7455) (width 0.25) (layer "B.Cu") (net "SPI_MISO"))
 (segment (start 3.0752 18.7455) (end 3.0866 18.7569) (width 0.25) (layer "B.Cu") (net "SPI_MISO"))
 (segment (start 2.3447 44.6647) (end 2.3447 22.7953) (width 0.25) (layer "B.Cu") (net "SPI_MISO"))
 (segment (start 1.9 3.36) (end 2.4278 3.8878) (width 0.25) (layer "B.Cu") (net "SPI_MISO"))
 (segment (start 4 46.32) (end 2.3447 44.6647) (width 0.25) (layer "B.Cu") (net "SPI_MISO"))
 (segment (start 3.0866 22.0534) (end 3.0866 18.7569) (width 0.25) (layer "B.Cu") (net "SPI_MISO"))
 (segment (start 5.2079 46.7741) (end 4.9827 46.9993) (width 0.25) (layer "F.Cu") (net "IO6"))
 (segment (start 4.9827 47.8773) (end 4 48.86) (width 0.25) (layer "F.Cu") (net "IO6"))
 (segment (start 4.9827 46.9993) (end 4.9827 47.27) (width 0.25) (layer "F.Cu") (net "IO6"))
 (segment (start 4.9827 47.27) (end 4.9827 47.8773) (width 0.25) (layer "F.Cu") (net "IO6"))
 (segment (start 0.8 12.253) (end 2.3007 12.253) (width 0.25) (layer "F.Cu") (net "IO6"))
 (segment (start 5.2079 15.1602) (end 5.2079 46.7741) (width 0.25) (layer "F.Cu") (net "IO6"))
 (segment (start 2.3007 12.253) (end 5.2079 15.1602) (width 0.25) (layer "F.Cu") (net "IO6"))
 (via (at 0.8 12.253) (size 0.8) (drill 0.3) (layers "F.Cu" "B.Cu") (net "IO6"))
 (segment (start 0.6 6.5) (end 0.6 13) (width 0.25) (layer "B.Cu") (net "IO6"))
 (segment (start 1.9 5.9) (end 0.6 6.5) (width 0.25) (layer "B.Cu") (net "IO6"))
 (segment (start 0.6 13) (end 0.8 12.253) (width 0.25) (layer "B.Cu") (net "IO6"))
 (segment (start 1.9302 8.4702) (end 3.0752 8.4702) (width 0.25) (layer "F.Cu") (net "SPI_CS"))
 (segment (start 1.9 8.44) (end 1.9302 8.4702) (width 0.25) (layer "F.Cu") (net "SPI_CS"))
 (segment (start 3.0752 8.4702) (end 3.0752 11.0714) (width 0.25) (layer "F.Cu") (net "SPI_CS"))
 (segment (start 5.6596 13.6558) (end 4.0017 11.9979) (width 0.25) (layer "F.Cu") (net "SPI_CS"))
 (segment (start 3.0752 11.0714) (end 4.0017 11.9979) (width 0.25) (layer "F.Cu") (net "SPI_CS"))
 (segment (start 4 51.4) (end 5.6596 49.7404) (width 0.25) (layer "F.Cu") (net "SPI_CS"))
 (segment (start 5.6596 49.7404) (end 5.6596 13.6558) (width 0.25) (layer "F.Cu") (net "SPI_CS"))
 (segment (start 0.7191 17.2409) (end 0.7191 24.2407) (width 0.25) (layer "F.Cu") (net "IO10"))
 (segment (start 1.9 16.06) (end 0.7191 17.2409) (width 0.25) (layer "F.Cu") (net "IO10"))
 (segment (start 0.7191 24.2407) (end 1.2552 24.7768) (width 0.25) (layer "F.Cu") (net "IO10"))
 (via (at 1.2552 24.7768) (size 0.8) (drill 0.3) (layers "F.Cu" "B.Cu") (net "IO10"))
 (segment (start 1.2552 51.1952) (end 4 53.94) (width 0.25) (layer "B.Cu") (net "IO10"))
 (segment (start 1.2552 24.7768) (end 1.2552 51.1952) (width 0.25) (layer "B.Cu") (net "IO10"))
 (segment (start 4 33.62) (end 4.66 33.62) (width 0.25) (layer "B.Cu") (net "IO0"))
 (segment (start 4.66 33.62) (end 17.14 21.14) (width 0.25) (layer "B.Cu") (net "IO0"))
 (segment (start 18.356 19.816) (end 18.356 21.804) (width 0.25) (layer "B.Cu") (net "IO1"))
 (segment (start 18.356 21.804) (end 4 36.16) (width 0.25) (layer "B.Cu") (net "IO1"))
 (segment (start 17.14 18.6) (end 18.356 19.816) (width 0.25) (layer "B.Cu") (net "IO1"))
 (segment (start 18.8424 17.7624) (end 18.8424 23.8576) (width 0.25) (layer "B.Cu") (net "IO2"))
 (segment (start 17.14 16.06) (end 18.8424 17.7624) (width 0.25) (layer "B.Cu") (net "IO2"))
 (segment (start 18.8424 23.8576) (end 4 38.7) (width 0.25) (layer "B.Cu") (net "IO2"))
 (segment (start 5.4814 31.2685) (end 5.4814 25.1786) (width 0.25) (layer "B.Cu") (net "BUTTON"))
 (segment (start 2.8 33.0639) (end 3.5139 32.35) (width 0.25) (layer "B.Cu") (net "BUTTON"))
 (segment (start 4 41.24) (end 2.8 40.04) (width 0.25) (layer "B.Cu") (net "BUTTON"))
 (segment (start 2.8 40.04) (end 2.8 33.0639) (width 0.25) (layer "B.Cu") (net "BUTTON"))
 (segment (start 3.5139 32.35) (end 4.3999 32.35) (width 0.25) (layer "B.Cu") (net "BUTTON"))
 (segment (start 5.4814 25.1786) (end 17.14 13.52) (width 0.25) (layer "B.Cu") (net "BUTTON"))
 (segment (start 4.3999 32.35) (end 5.4814 31.2685) (width 0.25) (layer "B.Cu") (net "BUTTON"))
 (segment (start 4 43.78) (end 19.328 28.452) (width 0.25) (layer "B.Cu") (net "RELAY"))
 (segment (start 19.328 28.452) (end 19.328 13.168) (width 0.25) (layer "B.Cu") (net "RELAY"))
 (segment (start 19.328 13.168) (end 17.14 10.98) (width 0.25) (layer "B.Cu") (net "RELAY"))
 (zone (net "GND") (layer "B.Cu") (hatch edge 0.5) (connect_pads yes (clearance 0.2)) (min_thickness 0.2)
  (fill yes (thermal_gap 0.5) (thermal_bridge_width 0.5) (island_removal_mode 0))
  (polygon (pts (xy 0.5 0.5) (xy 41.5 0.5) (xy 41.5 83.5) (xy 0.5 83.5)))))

